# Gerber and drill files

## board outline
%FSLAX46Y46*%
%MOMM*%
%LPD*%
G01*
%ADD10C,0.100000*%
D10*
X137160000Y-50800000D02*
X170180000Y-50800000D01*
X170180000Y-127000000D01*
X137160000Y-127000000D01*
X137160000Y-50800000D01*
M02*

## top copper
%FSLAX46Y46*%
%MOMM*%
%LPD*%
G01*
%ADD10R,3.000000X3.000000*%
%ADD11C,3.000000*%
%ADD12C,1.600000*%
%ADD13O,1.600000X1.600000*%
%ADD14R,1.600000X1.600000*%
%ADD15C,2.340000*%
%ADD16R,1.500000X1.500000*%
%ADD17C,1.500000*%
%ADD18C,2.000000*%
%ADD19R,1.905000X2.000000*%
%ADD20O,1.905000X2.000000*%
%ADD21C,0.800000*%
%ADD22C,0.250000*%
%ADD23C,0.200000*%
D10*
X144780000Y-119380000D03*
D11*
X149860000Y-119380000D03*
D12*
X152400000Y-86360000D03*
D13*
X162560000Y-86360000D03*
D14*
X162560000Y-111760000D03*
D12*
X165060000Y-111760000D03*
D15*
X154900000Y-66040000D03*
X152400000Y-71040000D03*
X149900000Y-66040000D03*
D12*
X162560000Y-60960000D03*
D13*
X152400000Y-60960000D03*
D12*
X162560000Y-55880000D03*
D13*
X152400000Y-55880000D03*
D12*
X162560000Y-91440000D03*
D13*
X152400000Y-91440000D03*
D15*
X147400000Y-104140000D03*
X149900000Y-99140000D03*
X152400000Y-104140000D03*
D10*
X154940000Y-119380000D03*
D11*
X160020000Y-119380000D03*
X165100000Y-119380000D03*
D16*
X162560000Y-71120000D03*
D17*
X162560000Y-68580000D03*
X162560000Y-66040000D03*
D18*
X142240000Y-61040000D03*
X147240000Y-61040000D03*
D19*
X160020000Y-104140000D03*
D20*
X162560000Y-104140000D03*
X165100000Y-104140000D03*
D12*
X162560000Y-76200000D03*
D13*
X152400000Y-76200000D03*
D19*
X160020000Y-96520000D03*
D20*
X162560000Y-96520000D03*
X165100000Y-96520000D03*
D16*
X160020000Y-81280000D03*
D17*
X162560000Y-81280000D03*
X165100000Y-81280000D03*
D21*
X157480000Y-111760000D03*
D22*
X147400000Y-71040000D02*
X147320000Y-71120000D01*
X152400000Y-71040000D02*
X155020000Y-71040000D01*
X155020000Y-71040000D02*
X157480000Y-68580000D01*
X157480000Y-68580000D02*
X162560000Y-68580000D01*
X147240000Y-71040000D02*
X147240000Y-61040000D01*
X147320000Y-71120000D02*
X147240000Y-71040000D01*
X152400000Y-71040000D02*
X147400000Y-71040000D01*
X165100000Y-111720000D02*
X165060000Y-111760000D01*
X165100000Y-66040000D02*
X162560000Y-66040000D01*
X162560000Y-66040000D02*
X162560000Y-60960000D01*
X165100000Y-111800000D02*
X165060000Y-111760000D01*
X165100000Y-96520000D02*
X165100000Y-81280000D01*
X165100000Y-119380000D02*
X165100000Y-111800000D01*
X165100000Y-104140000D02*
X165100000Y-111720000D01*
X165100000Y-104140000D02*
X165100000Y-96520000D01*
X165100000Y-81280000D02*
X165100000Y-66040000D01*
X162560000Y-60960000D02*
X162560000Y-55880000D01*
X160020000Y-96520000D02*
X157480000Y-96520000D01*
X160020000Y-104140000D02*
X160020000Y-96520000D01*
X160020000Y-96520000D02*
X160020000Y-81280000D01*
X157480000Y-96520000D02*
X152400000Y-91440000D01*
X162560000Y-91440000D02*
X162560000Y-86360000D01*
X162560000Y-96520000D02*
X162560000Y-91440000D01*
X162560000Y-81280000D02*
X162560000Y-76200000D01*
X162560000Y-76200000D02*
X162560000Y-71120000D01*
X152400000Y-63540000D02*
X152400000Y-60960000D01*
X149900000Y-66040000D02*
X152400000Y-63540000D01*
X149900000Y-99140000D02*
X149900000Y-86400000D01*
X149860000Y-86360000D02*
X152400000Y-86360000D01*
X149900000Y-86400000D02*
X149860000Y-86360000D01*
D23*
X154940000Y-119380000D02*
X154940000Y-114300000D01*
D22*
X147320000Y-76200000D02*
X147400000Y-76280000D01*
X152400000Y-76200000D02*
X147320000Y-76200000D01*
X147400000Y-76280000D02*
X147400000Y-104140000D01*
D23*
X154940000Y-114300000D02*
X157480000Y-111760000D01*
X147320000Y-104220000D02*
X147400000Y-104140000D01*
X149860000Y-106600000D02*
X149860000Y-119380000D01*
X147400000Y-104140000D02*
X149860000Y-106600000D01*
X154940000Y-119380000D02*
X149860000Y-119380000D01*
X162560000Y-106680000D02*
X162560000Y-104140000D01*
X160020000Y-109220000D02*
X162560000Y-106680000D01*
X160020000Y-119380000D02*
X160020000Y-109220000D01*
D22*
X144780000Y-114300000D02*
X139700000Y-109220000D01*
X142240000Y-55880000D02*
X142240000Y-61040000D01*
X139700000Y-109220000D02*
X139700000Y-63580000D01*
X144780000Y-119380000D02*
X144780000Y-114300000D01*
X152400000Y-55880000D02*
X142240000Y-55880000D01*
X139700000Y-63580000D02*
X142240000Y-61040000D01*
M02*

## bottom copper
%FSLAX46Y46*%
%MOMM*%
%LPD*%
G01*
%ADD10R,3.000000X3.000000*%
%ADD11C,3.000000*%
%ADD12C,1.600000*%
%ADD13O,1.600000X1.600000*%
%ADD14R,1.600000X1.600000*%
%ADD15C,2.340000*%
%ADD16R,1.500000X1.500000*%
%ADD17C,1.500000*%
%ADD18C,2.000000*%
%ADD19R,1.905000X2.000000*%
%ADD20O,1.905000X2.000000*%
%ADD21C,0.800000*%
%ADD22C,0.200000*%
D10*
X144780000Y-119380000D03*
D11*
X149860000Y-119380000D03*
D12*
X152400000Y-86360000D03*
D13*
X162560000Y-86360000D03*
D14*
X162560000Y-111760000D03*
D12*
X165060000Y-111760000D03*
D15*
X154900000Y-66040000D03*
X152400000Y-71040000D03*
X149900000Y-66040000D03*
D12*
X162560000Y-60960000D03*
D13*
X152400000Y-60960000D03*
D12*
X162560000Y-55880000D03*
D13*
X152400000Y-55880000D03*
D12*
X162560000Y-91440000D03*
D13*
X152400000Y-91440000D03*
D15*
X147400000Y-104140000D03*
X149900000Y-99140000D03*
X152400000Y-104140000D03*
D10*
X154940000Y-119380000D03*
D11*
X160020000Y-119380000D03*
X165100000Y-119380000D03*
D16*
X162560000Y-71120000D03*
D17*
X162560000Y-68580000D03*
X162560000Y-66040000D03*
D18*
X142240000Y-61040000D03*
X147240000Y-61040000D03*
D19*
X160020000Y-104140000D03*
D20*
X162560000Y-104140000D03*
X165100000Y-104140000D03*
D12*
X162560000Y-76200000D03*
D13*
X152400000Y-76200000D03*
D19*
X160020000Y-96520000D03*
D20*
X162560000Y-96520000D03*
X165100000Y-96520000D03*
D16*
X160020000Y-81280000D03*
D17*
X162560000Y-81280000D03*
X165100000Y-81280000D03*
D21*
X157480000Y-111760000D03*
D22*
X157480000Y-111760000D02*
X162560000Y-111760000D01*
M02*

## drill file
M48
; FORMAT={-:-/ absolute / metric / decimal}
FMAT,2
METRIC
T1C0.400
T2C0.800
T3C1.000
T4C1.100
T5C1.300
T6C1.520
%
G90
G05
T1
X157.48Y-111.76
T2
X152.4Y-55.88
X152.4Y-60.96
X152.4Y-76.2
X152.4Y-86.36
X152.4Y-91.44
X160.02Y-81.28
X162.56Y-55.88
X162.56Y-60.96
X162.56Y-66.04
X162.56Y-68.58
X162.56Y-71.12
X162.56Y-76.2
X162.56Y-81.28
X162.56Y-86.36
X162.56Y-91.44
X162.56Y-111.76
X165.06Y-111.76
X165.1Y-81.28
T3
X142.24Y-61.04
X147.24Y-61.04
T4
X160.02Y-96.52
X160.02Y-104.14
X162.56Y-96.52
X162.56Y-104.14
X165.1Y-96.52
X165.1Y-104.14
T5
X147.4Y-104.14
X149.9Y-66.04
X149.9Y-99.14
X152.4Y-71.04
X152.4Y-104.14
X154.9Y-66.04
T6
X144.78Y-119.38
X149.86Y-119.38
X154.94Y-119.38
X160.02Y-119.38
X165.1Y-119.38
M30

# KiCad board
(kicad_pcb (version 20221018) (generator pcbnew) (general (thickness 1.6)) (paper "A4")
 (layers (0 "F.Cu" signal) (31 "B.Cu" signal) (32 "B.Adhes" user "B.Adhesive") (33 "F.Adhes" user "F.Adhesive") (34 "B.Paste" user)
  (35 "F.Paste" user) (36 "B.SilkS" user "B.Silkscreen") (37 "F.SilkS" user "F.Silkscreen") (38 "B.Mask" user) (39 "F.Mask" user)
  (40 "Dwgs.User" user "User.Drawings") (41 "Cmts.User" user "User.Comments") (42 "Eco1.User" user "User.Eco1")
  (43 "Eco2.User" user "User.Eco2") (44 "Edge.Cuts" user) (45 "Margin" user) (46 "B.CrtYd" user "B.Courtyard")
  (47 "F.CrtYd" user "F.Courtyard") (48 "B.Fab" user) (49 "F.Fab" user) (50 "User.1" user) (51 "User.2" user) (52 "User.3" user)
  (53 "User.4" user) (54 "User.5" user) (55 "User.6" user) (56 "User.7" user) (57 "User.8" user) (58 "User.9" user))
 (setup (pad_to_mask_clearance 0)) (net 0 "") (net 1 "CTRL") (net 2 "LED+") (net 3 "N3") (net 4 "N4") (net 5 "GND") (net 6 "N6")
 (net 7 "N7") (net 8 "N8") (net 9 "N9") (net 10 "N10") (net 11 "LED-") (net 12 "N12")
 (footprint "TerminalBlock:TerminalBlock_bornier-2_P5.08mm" (layer "F.Cu") (at 144.78 119.38)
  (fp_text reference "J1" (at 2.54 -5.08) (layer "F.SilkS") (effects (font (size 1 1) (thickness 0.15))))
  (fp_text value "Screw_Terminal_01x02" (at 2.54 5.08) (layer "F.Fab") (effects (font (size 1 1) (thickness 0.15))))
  (pad "1" thru_hole rect (at 0 0) (size 3 3) (drill 1.52) (layers "*.Cu" "*.Mask") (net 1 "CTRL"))
  (pad "2" thru_hole circle (at 5.08 0) (size 3 3) (drill 1.52) (layers "*.Cu" "*.Mask") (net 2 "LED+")))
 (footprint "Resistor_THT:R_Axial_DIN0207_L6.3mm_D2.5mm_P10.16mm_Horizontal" (layer "F.Cu") (at 152.4 86.36)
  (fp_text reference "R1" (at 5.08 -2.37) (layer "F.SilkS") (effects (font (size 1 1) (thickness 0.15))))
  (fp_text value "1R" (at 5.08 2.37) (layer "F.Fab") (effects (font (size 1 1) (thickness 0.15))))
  (pad "1" thru_hole circle (at 0 0) (size 1.6 1.6) (drill 0.8) (layers "*.Cu" "*.Mask") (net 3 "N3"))
  (pad "2" thru_hole oval (at 10.16 0) (size 1.6 1.6) (drill 0.8) (layers "*.Cu" "*.Mask") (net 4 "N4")))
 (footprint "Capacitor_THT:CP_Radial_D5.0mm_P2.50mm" (layer "F.Cu") (at 162.56 111.76)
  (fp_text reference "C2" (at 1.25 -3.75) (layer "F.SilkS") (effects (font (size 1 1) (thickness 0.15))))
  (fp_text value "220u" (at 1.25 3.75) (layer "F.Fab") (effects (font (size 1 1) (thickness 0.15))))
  (pad "1" thru_hole rect (at 0 0) (size 1.6 1.6) (drill 0.8) (layers "*.Cu" "*.Mask") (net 2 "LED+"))
  (pad "2" thru_hole circle (at 2.5 0) (size 1.6 1.6) (drill 0.8) (layers "*.Cu" "*.Mask") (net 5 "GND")))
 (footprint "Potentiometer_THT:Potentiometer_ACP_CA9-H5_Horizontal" (layer "F.Cu") (at 154.9 66.04 -90)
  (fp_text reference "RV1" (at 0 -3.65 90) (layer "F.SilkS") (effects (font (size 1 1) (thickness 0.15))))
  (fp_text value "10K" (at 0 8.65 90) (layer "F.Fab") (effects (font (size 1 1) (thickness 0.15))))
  (pad "1" thru_hole circle (at 0 0 270) (size 2.34 2.34) (drill 1.3) (layers "*.Cu" "*.Mask") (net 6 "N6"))
  (pad "2" thru_hole circle (at 5 2.5 270) (size 2.34 2.34) (drill 1.3) (layers "*.Cu" "*.Mask") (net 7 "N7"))
  (pad "3" thru_hole circle (at 0 5 270) (size 2.34 2.34) (drill 1.3) (layers "*.Cu" "*.Mask") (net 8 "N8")))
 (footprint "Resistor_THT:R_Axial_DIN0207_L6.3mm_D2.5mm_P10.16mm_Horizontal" (layer "F.Cu") (at 162.56 60.96 180)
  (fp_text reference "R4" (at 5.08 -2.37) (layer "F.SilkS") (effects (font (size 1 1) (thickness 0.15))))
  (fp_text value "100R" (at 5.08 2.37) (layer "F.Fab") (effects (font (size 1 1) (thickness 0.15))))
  (pad "1" thru_hole circle (at 0 0 180) (size 1.6 1.6) (drill 0.8) (layers "*.Cu" "*.Mask") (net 5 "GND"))
  (pad "2" thru_hole oval (at 10.16 0 180) (size 1.6 1.6) (drill 0.8) (layers "*.Cu" "*.Mask") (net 8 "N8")))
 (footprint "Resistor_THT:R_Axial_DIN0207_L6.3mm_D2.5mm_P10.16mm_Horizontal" (layer "F.Cu") (at 162.56 55.88 180)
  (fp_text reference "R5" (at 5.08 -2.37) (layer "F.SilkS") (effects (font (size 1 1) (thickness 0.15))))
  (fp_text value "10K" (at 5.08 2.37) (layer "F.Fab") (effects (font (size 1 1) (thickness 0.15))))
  (pad "1" thru_hole circle (at 0 0 180) (size 1.6 1.6) (drill 0.8) (layers "*.Cu" "*.Mask") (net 5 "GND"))
  (pad "2" thru_hole oval (at 10.16 0 180) (size 1.6 1.6) (drill 0.8) (layers "*.Cu" "*.Mask") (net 1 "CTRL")))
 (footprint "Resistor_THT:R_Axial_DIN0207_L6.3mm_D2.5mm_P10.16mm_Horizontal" (layer "F.Cu") (at 162.56 91.44 180)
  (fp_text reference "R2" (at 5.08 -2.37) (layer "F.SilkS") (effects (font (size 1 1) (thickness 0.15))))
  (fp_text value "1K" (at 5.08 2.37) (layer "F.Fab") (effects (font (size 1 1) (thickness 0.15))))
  (pad "1" thru_hole circle (at 0 0 180) (size 1.6 1.6) (drill 0.8) (layers "*.Cu" "*.Mask") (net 4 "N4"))
  (pad "2" thru_hole oval (at 10.16 0 180) (size 1.6 1.6) (drill 0.8) (layers "*.Cu" "*.Mask") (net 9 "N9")))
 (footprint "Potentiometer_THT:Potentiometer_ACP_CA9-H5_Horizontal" (layer "F.Cu") (at 147.4 104.14 90)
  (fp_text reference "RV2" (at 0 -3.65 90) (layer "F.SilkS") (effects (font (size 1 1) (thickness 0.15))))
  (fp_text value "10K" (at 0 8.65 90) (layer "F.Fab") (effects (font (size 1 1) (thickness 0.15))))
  (pad "1" thru_hole circle (at 0 0 90) (size 2.34 2.34) (drill 1.3) (layers "*.Cu" "*.Mask") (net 2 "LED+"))
  (pad "2" thru_hole circle (at 5 2.5 90) (size 2.34 2.34) (drill 1.3) (layers "*.Cu" "*.Mask") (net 3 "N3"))
  (pad "3" thru_hole circle (at 0 5 90) (size 2.34 2.34) (drill 1.3) (layers "*.Cu" "*.Mask") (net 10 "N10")))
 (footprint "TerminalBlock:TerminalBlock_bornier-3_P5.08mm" (layer "F.Cu") (at 154.94 119.38)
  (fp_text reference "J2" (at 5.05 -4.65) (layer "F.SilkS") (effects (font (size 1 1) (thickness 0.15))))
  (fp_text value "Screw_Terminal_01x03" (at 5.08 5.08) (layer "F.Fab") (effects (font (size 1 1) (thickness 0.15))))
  (pad "1" thru_hole rect (at 0 0) (size 3 3) (drill 1.52) (layers "*.Cu" "*.Mask") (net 2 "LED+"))
  (pad "2" thru_hole circle (at 5.08 0) (size 3 3) (drill 1.52) (layers "*.Cu" "*.Mask") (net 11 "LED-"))
  (pad "3" thru_hole circle (at 10.16 0) (size 3 3) (drill 1.52) (layers "*.Cu" "*.Mask") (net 5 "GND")))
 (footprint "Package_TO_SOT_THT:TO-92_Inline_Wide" (layer "F.Cu") (at 162.56 71.12 90)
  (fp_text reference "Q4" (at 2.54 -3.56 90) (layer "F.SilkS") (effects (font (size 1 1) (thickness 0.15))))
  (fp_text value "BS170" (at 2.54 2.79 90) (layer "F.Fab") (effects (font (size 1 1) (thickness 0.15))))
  (pad "1" thru_hole rect (at 0 0 90) (size 1.5 1.5) (drill 0.8) (layers "*.Cu" "*.Mask") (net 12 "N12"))
  (pad "2" thru_hole circle (at 2.54 0 90) (size 1.5 1.5) (drill 0.8) (layers "*.Cu" "*.Mask") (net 7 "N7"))
  (pad "3" thru_hole circle (at 5.08 0 90) (size 1.5 1.5) (drill 0.8) (layers "*.Cu" "*.Mask") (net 5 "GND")))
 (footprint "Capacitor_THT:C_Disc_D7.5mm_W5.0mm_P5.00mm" (layer "F.Cu") (at 142.24 61.04)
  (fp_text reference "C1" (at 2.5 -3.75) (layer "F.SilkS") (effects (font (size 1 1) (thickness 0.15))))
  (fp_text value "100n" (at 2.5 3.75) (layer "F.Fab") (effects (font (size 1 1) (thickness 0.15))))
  (pad "1" thru_hole circle (at 0 0) (size 2 2) (drill 1) (layers "*.Cu" "*.Mask") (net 1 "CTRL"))
  (pad "2" thru_hole circle (at 5 0) (size 2 2) (drill 1) (layers "*.Cu" "*.Mask") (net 7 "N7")))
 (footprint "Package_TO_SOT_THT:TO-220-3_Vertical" (layer "F.Cu") (at 160.02 104.14)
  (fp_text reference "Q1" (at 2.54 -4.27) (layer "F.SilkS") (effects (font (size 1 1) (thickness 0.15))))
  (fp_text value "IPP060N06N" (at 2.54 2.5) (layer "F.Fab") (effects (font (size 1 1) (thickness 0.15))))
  (pad "1" thru_hole rect (at 0 0) (size 1.905 2) (drill 1.1) (layers "*.Cu" "*.Mask") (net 9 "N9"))
  (pad "2" thru_hole oval (at 2.54 0) (size 1.905 2) (drill 1.1) (layers "*.Cu" "*.Mask") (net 11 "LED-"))
  (pad "3" thru_hole oval (at 5.08 0) (size 1.905 2) (drill 1.1) (layers "*.Cu" "*.Mask") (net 5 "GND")))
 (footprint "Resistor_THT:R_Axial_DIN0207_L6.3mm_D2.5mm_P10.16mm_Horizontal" (layer "F.Cu") (at 162.56 76.2 180)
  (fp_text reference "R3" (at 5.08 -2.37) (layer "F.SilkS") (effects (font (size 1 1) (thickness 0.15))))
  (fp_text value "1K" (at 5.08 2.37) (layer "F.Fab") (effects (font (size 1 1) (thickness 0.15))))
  (pad "1" thru_hole circle (at 0 0 180) (size 1.6 1.6) (drill 0.8) (layers "*.Cu" "*.Mask") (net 12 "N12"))
  (pad "2" thru_hole oval (at 10.16 0 180) (size 1.6 1.6) (drill 0.8) (layers "*.Cu" "*.Mask") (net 2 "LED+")))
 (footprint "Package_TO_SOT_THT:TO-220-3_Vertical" (layer "F.Cu") (at 160.02 96.52)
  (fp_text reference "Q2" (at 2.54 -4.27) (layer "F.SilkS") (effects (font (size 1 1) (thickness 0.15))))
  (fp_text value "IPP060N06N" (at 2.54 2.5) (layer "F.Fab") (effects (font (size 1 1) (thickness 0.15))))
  (pad "1" thru_hole rect (at 0 0) (size 1.905 2) (drill 1.1) (layers "*.Cu" "*.Mask") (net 9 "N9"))
  (pad "2" thru_hole oval (at 2.54 0) (size 1.905 2) (drill 1.1) (layers "*.Cu" "*.Mask") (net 4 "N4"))
  (pad "3" thru_hole oval (at 5.08 0) (size 1.905 2) (drill 1.1) (layers "*.Cu" "*.Mask") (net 5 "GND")))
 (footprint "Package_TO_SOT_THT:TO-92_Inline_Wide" (layer "F.Cu") (at 160.02 81.28)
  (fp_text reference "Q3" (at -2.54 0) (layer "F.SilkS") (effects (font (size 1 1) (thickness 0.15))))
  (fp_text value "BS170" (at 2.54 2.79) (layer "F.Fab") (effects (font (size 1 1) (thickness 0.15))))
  (pad "1" thru_hole rect (at 0 0) (size 1.5 1.5) (drill 0.8) (layers "*.Cu" "*.Mask") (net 9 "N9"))
  (pad "2" thru_hole circle (at 2.54 0) (size 1.5 1.5) (drill 0.8) (layers "*.Cu" "*.Mask") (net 12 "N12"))
  (pad "3" thru_hole circle (at 5.08 0) (size 1.5 1.5) (drill 0.8) (layers "*.Cu" "*.Mask") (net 5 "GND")))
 (gr_rect (start 137.16 50.8) (end 170.18 127) (stroke (width 0.1) (type default)) (fill none) (layer "Edge.Cuts"))
 (segment (start 147.4 71.04) (end 147.32 71.12) (width 0.25) (layer "F.Cu") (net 7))
 (segment (start 152.4 71.04) (end 155.02 71.04) (width 0.25) (layer "F.Cu") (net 7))
 (segment (start 155.02 71.04) (end 157.48 68.58) (width 0.25) (layer "F.Cu") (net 7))
 (segment (start 157.48 68.58) (end 162.56 68.58) (width 0.25) (layer "F.Cu") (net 7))
 (segment (start 147.24 71.04) (end 147.24 61.04) (width 0.25) (layer "F.Cu") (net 7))
 (segment (start 147.32 71.12) (end 147.24 71.04) (width 0.25) (layer "F.Cu") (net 7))
 (segment (start 152.4 71.04) (end 147.4 71.04) (width 0.25) (layer "F.Cu") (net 7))
 (segment (start 165.1 111.72) (end 165.06 111.76) (width 0.25) (layer "F.Cu") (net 5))
 (segment (start 165.1 66.04) (end 162.56 66.04) (width 0.25) (layer "F.Cu") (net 5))
 (segment (start 162.56 66.04) (end 162.56 60.96) (width 0.25) (layer "F.Cu") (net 5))
 (segment (start 165.1 111.8) (end 165.06 111.76) (width 0.25) (layer "F.Cu") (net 5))
 (segment (start 165.1 96.52) (end 165.1 81.28) (width 0.25) (layer "F.Cu") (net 5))
 (segment (start 165.1 119.38) (end 165.1 111.8) (width 0.25) (layer "F.Cu") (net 5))
 (segment (start 165.1 104.14) (end 165.1 111.72) (width 0.25) (layer "F.Cu") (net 5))
 (segment (start 165.1 104.14) (end 165.1 96.52) (width 0.25) (layer "F.Cu") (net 5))
 (segment (start 165.1 81.28) (end 165.1 66.04) (width 0.25) (layer "F.Cu") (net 5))
 (segment (start 162.56 60.96) (end 162.56 55.88) (width 0.25) (layer "F.Cu") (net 5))
 (segment (start 160.02 96.52) (end 157.48 96.52) (width 0.25) (layer "F.Cu") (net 9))
 (segment (start 160.02 104.14) (end 160.02 96.52) (width 0.25) (layer "F.Cu") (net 9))
 (segment (start 160.02 96.52) (end 160.02 81.28) (width 0.25) (layer "F.Cu") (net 9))
 (segment (start 157.48 96.52) (end 152.4 91.44) (width 0.25) (layer "F.Cu") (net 9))
 (segment (start 162.56 91.44) (end 162.56 86.36) (width 0.25) (layer "F.Cu") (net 4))
 (segment (start 162.56 96.52) (end 162.56 91.44) (width 0.25) (layer "F.Cu") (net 4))
 (segment (start 162.56 81.28) (end 162.56 76.2) (width 0.25) (layer "F.Cu") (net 12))
 (segment (start 162.56 76.2) (end 162.56 71.12) (width 0.25) (layer "F.Cu") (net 12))
 (segment (start 152.4 63.54) (end 152.4 60.96) (width 0.25) (layer "F.Cu") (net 8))
 (segment (start 149.9 66.04) (end 152.4 63.54) (width 0.25) (layer "F.Cu") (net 8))
 (segment (start 149.9 99.14) (end 149.9 86.4) (width 0.25) (layer "F.Cu") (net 3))
 (segment (start 149.86 86.36) (end 152.4 86.36) (width 0.25) (layer "F.Cu") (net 3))
 (segment (start 149.9 86.4) (end 149.86 86.36) (width 0.25) (layer "F.Cu") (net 3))
 (segment (start 154.94 119.38) (end 154.94 114.3) (width 0.2) (layer "F.Cu") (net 2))
 (segment (start 147.32 76.2) (end 147.4 76.28) (width 0.25) (layer "F.Cu") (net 2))
 (segment (start 152.4 76.2) (end 147.32 76.2) (width 0.25) (layer "F.Cu") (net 2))
 (segment (start 147.4 76.28) (end 147.4 104.14) (width 0.25) (layer "F.Cu") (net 2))
 (segment (start 154.94 114.3) (end 157.48 111.76) (width 0.2) (layer "F.Cu") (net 2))
 (segment (start 147.32 104.22) (end 147.4 104.14) (width 0.2) (layer "F.Cu") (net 2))
 (segment (start 149.86 106.6) (end 149.86 119.38) (width 0.2) (layer "F.Cu") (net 2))
 (segment (start 147.4 104.14) (end 149.86 106.6) (width 0.2) (layer "F.Cu") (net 2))
 (segment (start 154.94 119.38) (end 149.86 119.38) (width 0.2) (layer "F.Cu") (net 2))
 (via (at 157.48 111.76) (size 0.8) (drill 0.4) (layers "F.Cu" "B.Cu") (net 2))
 (segment (start 157.48 111.76) (end 162.56 111.76) (width 0.2) (layer "B.Cu") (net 2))
 (segment (start 162.56 106.68) (end 162.56 104.14) (width 0.2) (layer "F.Cu") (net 11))
 (segment (start 160.02 109.22) (end 162.56 106.68) (width 0.2) (layer "F.Cu") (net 11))
 (segment (start 160.02 119.38) (end 160.02 109.22) (width 0.2) (layer "F.Cu") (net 11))
 (segment (start 144.78 114.3) (end 139.7 109.22) (width 0.25) (layer "F.Cu") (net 1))
 (segment (start 142.24 55.88) (end 142.24 61.04) (width 0.25) (layer "F.Cu") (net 1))
 (segment (start 139.7 109.22) (end 139.7 63.58) (width 0.25) (layer "F.Cu") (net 1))
 (segment (start 144.78 119.38) (end 144.78 114.3) (width 0.25) (layer "F.Cu") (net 1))
 (segment (start 152.4 55.88) (end 142.24 55.88) (width 0.25) (layer "F.Cu") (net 1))
 (segment (start 139.7 63.58) (end 142.24 61.04) (width 0.25) (layer "F.Cu") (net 1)))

